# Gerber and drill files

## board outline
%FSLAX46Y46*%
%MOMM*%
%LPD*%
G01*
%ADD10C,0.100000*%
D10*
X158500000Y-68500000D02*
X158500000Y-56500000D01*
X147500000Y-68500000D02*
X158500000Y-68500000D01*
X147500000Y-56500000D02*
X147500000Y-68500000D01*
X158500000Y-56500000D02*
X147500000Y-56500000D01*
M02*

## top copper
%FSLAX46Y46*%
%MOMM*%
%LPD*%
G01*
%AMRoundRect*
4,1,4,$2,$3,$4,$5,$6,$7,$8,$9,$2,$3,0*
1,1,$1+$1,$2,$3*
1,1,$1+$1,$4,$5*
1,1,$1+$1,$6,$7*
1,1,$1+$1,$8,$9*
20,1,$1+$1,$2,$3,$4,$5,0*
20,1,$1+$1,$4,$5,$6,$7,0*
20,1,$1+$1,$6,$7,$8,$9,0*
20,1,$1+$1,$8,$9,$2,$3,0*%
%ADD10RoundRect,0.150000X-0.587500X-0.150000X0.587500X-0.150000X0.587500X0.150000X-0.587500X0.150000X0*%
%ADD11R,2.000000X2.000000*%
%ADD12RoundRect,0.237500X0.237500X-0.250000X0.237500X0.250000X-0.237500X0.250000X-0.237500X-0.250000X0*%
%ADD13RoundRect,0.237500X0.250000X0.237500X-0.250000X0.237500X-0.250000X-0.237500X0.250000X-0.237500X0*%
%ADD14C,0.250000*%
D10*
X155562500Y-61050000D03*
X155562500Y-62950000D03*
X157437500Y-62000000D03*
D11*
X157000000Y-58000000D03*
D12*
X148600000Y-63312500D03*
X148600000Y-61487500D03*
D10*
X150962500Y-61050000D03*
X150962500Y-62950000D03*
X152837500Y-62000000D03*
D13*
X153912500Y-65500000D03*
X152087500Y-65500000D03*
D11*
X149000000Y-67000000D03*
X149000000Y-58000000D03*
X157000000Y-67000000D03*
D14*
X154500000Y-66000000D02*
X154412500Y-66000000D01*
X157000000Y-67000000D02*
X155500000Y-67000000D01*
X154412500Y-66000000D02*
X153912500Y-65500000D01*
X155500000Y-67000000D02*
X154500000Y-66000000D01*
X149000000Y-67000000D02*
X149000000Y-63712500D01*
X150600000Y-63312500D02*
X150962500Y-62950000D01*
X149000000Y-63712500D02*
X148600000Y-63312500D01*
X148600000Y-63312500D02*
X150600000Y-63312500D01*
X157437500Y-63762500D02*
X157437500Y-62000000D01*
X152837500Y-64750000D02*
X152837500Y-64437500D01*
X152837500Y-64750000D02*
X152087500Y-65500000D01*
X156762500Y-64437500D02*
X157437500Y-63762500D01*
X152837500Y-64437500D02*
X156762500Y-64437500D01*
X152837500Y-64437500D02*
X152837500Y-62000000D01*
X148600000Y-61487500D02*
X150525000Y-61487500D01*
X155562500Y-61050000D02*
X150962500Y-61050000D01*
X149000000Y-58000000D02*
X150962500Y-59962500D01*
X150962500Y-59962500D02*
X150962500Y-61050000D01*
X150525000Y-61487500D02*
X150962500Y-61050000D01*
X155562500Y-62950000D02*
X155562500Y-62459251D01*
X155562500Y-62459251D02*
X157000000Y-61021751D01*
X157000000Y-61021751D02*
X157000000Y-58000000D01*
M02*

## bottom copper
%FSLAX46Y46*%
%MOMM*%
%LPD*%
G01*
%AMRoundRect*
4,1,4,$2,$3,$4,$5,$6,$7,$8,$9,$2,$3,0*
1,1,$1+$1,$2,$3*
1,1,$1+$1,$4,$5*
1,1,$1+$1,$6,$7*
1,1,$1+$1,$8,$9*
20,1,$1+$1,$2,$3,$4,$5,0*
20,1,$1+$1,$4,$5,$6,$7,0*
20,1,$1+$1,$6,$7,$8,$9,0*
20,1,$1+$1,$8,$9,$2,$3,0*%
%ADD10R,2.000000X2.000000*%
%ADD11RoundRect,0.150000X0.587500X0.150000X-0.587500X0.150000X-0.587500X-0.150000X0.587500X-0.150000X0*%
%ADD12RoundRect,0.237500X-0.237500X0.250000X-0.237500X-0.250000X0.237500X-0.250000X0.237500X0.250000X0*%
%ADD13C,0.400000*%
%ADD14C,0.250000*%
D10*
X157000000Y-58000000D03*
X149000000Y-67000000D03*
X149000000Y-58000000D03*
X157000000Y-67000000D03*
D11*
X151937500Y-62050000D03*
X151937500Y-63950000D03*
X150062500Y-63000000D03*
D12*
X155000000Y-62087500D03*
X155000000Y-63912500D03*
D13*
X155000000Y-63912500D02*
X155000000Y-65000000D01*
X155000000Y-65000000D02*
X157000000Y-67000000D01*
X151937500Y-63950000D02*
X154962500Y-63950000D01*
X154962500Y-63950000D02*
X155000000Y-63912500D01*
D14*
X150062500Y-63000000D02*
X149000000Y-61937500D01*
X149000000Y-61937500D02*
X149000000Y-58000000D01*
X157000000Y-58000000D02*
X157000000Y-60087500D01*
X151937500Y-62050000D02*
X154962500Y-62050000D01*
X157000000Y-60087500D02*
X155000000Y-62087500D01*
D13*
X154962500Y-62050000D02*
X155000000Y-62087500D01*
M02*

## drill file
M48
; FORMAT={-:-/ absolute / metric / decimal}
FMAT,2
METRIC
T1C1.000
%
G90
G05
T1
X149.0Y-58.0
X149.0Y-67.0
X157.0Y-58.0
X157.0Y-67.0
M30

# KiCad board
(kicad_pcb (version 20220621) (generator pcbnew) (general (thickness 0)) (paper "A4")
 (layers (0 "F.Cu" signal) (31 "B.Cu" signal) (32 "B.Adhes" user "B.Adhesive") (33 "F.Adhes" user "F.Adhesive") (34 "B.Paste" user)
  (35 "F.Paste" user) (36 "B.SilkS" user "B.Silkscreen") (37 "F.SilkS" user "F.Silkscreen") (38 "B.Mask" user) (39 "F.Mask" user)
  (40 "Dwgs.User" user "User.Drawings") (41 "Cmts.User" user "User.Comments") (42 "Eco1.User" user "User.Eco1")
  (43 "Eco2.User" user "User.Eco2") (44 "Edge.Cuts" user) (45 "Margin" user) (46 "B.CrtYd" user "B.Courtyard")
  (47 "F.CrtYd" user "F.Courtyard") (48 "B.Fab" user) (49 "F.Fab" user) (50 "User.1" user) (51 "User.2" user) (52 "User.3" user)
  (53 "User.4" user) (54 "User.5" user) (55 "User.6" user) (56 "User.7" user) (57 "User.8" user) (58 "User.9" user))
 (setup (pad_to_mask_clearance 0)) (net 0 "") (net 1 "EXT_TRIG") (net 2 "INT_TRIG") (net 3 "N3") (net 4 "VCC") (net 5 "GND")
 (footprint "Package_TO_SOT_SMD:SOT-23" (layer "F.Cu") (at 156.5 62)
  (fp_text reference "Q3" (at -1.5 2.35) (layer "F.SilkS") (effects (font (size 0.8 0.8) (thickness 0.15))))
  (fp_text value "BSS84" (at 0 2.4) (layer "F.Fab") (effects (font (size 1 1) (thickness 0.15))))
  (pad "1" smd roundrect (at -0.9375 -0.95) (size 1.475 0.6) (layers "F.Cu" "F.Paste" "F.Mask") (roundrect_rratio 0.25) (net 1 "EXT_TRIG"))
  (pad "2" smd roundrect (at -0.9375 0.95) (size 1.475 0.6) (layers "F.Cu" "F.Paste" "F.Mask") (roundrect_rratio 0.25) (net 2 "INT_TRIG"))
  (pad "3" smd roundrect (at 0.9375 0) (size 1.475 0.6) (layers "F.Cu" "F.Paste" "F.Mask") (roundrect_rratio 0.25) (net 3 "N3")))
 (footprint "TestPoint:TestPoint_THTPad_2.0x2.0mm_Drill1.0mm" (layer "F.Cu") (at 157 58)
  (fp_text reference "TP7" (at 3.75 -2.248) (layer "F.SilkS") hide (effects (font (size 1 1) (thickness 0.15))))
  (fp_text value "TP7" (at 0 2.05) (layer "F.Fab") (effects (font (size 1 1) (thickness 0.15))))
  (pad "1" thru_hole rect (at 0 0) (size 2 2) (drill 1) (layers *.Cu *.Mask) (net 2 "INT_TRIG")))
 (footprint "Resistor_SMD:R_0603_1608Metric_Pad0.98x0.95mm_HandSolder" (layer "F.Cu") (at 148.6 62.4 90)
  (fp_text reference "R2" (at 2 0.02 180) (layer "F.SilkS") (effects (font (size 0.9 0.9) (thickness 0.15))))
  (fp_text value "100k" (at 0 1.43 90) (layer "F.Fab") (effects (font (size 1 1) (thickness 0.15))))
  (pad "1" smd roundrect (at -0.9125 0 90) (size 0.975 0.95) (layers "F.Cu" "F.Paste" "F.Mask") (roundrect_rratio 0.25) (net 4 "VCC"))
  (pad "2" smd roundrect (at 0.9125 0 90) (size 0.975 0.95) (layers "F.Cu" "F.Paste" "F.Mask") (roundrect_rratio 0.25) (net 1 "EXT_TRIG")))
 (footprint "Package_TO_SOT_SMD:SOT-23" (layer "F.Cu") (at 151.9 62)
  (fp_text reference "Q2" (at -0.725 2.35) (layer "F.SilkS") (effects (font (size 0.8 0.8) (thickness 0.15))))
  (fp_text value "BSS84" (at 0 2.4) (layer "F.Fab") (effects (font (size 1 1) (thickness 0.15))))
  (pad "1" smd roundrect (at -0.9375 -0.95) (size 1.475 0.6) (layers "F.Cu" "F.Paste" "F.Mask") (roundrect_rratio 0.25) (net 1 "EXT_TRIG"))
  (pad "2" smd roundrect (at -0.9375 0.95) (size 1.475 0.6) (layers "F.Cu" "F.Paste" "F.Mask") (roundrect_rratio 0.25) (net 4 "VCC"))
  (pad "3" smd roundrect (at 0.9375 0) (size 1.475 0.6) (layers "F.Cu" "F.Paste" "F.Mask") (roundrect_rratio 0.25) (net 3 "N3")))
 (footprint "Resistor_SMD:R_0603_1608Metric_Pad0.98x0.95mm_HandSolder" (layer "F.Cu") (at 153 65.5 180)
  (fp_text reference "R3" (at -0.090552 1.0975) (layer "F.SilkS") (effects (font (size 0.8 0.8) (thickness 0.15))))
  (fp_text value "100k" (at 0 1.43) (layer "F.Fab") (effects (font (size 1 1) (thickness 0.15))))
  (pad "1" smd roundrect (at -0.9125 0 180) (size 0.975 0.95) (layers "F.Cu" "F.Paste" "F.Mask") (roundrect_rratio 0.25) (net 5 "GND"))
  (pad "2" smd roundrect (at 0.9125 0 180) (size 0.975 0.95) (layers "F.Cu" "F.Paste" "F.Mask") (roundrect_rratio 0.25) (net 3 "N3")))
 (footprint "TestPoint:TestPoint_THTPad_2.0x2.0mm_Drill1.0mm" (layer "F.Cu") (at 149 67)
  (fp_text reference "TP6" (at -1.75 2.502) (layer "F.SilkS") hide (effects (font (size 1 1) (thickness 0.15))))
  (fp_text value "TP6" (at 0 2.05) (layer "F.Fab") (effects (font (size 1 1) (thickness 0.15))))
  (pad "1" thru_hole rect (at 0 0) (size 2 2) (drill 1) (layers *.Cu *.Mask) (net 4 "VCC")))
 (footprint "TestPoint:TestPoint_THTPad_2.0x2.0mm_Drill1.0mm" (layer "F.Cu") (at 149 58)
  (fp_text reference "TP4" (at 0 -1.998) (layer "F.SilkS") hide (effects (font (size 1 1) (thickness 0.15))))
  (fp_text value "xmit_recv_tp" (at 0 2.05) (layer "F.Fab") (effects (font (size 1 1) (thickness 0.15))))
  (pad "1" thru_hole rect (at 0 0) (size 2 2) (drill 1) (layers *.Cu *.Mask) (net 1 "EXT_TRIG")))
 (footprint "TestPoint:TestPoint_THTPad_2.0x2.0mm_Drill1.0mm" (layer "F.Cu") (at 157 67)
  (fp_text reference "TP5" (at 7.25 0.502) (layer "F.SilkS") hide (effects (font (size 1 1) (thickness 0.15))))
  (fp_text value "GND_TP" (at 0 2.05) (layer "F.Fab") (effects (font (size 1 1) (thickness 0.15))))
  (pad "1" thru_hole rect (at 0 0) (size 2 2) (drill 1) (layers *.Cu *.Mask) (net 5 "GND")))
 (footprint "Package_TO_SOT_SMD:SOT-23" (layer "B.Cu") (at 151 63 180)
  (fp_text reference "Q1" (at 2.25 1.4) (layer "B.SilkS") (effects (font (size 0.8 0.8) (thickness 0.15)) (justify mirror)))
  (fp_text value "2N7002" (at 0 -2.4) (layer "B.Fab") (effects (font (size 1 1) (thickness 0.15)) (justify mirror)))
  (pad "1" smd roundrect (at -0.9375 0.95 180) (size 1.475 0.6) (layers "B.Cu" "B.Paste" "B.Mask") (roundrect_rratio 0.25)
   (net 2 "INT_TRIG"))
  (pad "2" smd roundrect (at -0.9375 -0.95 180) (size 1.475 0.6) (layers "B.Cu" "B.Paste" "B.Mask") (roundrect_rratio 0.25) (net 5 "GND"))
  (pad "3" smd roundrect (at 0.9375 0 180) (size 1.475 0.6) (layers "B.Cu" "B.Paste" "B.Mask") (roundrect_rratio 0.25) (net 1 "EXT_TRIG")))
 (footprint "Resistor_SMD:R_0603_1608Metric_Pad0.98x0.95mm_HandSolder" (layer "B.Cu") (at 155 63 -90)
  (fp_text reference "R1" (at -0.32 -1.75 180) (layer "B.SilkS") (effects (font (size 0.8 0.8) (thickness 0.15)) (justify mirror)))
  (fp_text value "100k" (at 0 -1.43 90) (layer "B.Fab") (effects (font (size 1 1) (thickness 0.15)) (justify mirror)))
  (pad "1" smd roundrect (at -0.9125 0 270) (size 0.975 0.95) (layers "B.Cu" "B.Paste" "B.Mask") (roundrect_rratio 0.25) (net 2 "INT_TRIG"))
  (pad "2" smd roundrect (at 0.9125 0 270) (size 0.975 0.95) (layers "B.Cu" "B.Paste" "B.Mask") (roundrect_rratio 0.25) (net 5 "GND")))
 (gr_line (start 158.5 68.5) (end 158.5 56.5) (stroke (width 0.1) (type default)) (layer "Edge.Cuts"))
 (gr_line (start 147.5 68.5) (end 158.5 68.5) (stroke (width 0.1) (type default)) (layer "Edge.Cuts"))
 (gr_line (start 147.5 56.5) (end 147.5 68.5) (stroke (width 0.1) (type default)) (layer "Edge.Cuts"))
 (gr_line (start 158.5 56.5) (end 147.5 56.5) (stroke (width 0.1) (type default)) (layer "Edge.Cuts"))
 (segment (start 154.5 66) (end 154.4125 66) (width 0.25) (layer "F.Cu") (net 5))
 (segment (start 157 67) (end 155.5 67) (width 0.25) (layer "F.Cu") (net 5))
 (segment (start 154.4125 66) (end 153.9125 65.5) (width 0.25) (layer "F.Cu") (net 5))
 (segment (start 155.5 67) (end 154.5 66) (width 0.25) (layer "F.Cu") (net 5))
 (segment (start 155 63.9125) (end 155 65) (width 0.4) (layer "B.Cu") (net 5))
 (segment (start 155 65) (end 157 67) (width 0.4) (layer "B.Cu") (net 5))
 (segment (start 151.9375 63.95) (end 154.9625 63.95) (width 0.4) (layer "B.Cu") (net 5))
 (segment (start 154.9625 63.95) (end 155 63.9125) (width 0.4) (layer "B.Cu") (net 5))
 (segment (start 149 67) (end 149 63.7125) (width 0.25) (layer "F.Cu") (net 4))
 (segment (start 150.6 63.3125) (end 150.9625 62.95) (width 0.25) (layer "F.Cu") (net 4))
 (segment (start 149 63.7125) (end 148.6 63.3125) (width 0.25) (layer "F.Cu") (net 4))
 (segment (start 148.6 63.3125) (end 150.6 63.3125) (width 0.25) (layer "F.Cu") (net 4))
 (segment (start 157.4375 63.7625) (end 157.4375 62) (width 0.25) (layer "F.Cu") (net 3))
 (segment (start 152.8375 64.75) (end 152.8375 64.4375) (width 0.25) (layer "F.Cu") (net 3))
 (segment (start 152.8375 64.75) (end 152.0875 65.5) (width 0.25) (layer "F.Cu") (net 3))
 (segment (start 156.7625 64.4375) (end 157.4375 63.7625) (width 0.25) (layer "F.Cu") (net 3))
 (segment (start 152.8375 64.4375) (end 156.7625 64.4375) (width 0.25) (layer "F.Cu") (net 3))
 (segment (start 152.8375 64.4375) (end 152.8375 62) (width 0.25) (layer "F.Cu") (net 3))
 (segment (start 148.6 61.4875) (end 150.525 61.4875) (width 0.25) (layer "F.Cu") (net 1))
 (segment (start 155.5625 61.05) (end 150.9625 61.05) (width 0.25) (layer "F.Cu") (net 1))
 (segment (start 149 58) (end 150.9625 59.9625) (width 0.25) (layer "F.Cu") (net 1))
 (segment (start 150.9625 59.9625) (end 150.9625 61.05) (width 0.25) (layer "F.Cu") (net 1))
 (segment (start 150.525 61.4875) (end 150.9625 61.05) (width 0.25) (layer "F.Cu") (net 1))
 (segment (start 150.0625 63) (end 149 61.9375) (width 0.25) (layer "B.Cu") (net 1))
 (segment (start 149 61.9375) (end 149 58) (width 0.25) (layer "B.Cu") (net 1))
 (segment (start 155.5625 62.95) (end 155.5625 62.459251) (width 0.25) (layer "F.Cu") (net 2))
 (segment (start 155.5625 62.459251) (end 157 61.021751) (width 0.25) (layer "F.Cu") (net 2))
 (segment (start 157 61.021751) (end 157 58) (width 0.25) (layer "F.Cu") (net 2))
 (segment (start 157 58) (end 157 60.0875) (width 0.25) (layer "B.Cu") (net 2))
 (segment (start 151.9375 62.05) (end 154.9625 62.05) (width 0.25) (layer "B.Cu") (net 2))
 (segment (start 157 60.0875) (end 155 62.0875) (width 0.25) (layer "B.Cu") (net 2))
 (segment (start 154.9625 62.05) (end 155 62.0875) (width 0.4) (layer "B.Cu") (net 2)))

